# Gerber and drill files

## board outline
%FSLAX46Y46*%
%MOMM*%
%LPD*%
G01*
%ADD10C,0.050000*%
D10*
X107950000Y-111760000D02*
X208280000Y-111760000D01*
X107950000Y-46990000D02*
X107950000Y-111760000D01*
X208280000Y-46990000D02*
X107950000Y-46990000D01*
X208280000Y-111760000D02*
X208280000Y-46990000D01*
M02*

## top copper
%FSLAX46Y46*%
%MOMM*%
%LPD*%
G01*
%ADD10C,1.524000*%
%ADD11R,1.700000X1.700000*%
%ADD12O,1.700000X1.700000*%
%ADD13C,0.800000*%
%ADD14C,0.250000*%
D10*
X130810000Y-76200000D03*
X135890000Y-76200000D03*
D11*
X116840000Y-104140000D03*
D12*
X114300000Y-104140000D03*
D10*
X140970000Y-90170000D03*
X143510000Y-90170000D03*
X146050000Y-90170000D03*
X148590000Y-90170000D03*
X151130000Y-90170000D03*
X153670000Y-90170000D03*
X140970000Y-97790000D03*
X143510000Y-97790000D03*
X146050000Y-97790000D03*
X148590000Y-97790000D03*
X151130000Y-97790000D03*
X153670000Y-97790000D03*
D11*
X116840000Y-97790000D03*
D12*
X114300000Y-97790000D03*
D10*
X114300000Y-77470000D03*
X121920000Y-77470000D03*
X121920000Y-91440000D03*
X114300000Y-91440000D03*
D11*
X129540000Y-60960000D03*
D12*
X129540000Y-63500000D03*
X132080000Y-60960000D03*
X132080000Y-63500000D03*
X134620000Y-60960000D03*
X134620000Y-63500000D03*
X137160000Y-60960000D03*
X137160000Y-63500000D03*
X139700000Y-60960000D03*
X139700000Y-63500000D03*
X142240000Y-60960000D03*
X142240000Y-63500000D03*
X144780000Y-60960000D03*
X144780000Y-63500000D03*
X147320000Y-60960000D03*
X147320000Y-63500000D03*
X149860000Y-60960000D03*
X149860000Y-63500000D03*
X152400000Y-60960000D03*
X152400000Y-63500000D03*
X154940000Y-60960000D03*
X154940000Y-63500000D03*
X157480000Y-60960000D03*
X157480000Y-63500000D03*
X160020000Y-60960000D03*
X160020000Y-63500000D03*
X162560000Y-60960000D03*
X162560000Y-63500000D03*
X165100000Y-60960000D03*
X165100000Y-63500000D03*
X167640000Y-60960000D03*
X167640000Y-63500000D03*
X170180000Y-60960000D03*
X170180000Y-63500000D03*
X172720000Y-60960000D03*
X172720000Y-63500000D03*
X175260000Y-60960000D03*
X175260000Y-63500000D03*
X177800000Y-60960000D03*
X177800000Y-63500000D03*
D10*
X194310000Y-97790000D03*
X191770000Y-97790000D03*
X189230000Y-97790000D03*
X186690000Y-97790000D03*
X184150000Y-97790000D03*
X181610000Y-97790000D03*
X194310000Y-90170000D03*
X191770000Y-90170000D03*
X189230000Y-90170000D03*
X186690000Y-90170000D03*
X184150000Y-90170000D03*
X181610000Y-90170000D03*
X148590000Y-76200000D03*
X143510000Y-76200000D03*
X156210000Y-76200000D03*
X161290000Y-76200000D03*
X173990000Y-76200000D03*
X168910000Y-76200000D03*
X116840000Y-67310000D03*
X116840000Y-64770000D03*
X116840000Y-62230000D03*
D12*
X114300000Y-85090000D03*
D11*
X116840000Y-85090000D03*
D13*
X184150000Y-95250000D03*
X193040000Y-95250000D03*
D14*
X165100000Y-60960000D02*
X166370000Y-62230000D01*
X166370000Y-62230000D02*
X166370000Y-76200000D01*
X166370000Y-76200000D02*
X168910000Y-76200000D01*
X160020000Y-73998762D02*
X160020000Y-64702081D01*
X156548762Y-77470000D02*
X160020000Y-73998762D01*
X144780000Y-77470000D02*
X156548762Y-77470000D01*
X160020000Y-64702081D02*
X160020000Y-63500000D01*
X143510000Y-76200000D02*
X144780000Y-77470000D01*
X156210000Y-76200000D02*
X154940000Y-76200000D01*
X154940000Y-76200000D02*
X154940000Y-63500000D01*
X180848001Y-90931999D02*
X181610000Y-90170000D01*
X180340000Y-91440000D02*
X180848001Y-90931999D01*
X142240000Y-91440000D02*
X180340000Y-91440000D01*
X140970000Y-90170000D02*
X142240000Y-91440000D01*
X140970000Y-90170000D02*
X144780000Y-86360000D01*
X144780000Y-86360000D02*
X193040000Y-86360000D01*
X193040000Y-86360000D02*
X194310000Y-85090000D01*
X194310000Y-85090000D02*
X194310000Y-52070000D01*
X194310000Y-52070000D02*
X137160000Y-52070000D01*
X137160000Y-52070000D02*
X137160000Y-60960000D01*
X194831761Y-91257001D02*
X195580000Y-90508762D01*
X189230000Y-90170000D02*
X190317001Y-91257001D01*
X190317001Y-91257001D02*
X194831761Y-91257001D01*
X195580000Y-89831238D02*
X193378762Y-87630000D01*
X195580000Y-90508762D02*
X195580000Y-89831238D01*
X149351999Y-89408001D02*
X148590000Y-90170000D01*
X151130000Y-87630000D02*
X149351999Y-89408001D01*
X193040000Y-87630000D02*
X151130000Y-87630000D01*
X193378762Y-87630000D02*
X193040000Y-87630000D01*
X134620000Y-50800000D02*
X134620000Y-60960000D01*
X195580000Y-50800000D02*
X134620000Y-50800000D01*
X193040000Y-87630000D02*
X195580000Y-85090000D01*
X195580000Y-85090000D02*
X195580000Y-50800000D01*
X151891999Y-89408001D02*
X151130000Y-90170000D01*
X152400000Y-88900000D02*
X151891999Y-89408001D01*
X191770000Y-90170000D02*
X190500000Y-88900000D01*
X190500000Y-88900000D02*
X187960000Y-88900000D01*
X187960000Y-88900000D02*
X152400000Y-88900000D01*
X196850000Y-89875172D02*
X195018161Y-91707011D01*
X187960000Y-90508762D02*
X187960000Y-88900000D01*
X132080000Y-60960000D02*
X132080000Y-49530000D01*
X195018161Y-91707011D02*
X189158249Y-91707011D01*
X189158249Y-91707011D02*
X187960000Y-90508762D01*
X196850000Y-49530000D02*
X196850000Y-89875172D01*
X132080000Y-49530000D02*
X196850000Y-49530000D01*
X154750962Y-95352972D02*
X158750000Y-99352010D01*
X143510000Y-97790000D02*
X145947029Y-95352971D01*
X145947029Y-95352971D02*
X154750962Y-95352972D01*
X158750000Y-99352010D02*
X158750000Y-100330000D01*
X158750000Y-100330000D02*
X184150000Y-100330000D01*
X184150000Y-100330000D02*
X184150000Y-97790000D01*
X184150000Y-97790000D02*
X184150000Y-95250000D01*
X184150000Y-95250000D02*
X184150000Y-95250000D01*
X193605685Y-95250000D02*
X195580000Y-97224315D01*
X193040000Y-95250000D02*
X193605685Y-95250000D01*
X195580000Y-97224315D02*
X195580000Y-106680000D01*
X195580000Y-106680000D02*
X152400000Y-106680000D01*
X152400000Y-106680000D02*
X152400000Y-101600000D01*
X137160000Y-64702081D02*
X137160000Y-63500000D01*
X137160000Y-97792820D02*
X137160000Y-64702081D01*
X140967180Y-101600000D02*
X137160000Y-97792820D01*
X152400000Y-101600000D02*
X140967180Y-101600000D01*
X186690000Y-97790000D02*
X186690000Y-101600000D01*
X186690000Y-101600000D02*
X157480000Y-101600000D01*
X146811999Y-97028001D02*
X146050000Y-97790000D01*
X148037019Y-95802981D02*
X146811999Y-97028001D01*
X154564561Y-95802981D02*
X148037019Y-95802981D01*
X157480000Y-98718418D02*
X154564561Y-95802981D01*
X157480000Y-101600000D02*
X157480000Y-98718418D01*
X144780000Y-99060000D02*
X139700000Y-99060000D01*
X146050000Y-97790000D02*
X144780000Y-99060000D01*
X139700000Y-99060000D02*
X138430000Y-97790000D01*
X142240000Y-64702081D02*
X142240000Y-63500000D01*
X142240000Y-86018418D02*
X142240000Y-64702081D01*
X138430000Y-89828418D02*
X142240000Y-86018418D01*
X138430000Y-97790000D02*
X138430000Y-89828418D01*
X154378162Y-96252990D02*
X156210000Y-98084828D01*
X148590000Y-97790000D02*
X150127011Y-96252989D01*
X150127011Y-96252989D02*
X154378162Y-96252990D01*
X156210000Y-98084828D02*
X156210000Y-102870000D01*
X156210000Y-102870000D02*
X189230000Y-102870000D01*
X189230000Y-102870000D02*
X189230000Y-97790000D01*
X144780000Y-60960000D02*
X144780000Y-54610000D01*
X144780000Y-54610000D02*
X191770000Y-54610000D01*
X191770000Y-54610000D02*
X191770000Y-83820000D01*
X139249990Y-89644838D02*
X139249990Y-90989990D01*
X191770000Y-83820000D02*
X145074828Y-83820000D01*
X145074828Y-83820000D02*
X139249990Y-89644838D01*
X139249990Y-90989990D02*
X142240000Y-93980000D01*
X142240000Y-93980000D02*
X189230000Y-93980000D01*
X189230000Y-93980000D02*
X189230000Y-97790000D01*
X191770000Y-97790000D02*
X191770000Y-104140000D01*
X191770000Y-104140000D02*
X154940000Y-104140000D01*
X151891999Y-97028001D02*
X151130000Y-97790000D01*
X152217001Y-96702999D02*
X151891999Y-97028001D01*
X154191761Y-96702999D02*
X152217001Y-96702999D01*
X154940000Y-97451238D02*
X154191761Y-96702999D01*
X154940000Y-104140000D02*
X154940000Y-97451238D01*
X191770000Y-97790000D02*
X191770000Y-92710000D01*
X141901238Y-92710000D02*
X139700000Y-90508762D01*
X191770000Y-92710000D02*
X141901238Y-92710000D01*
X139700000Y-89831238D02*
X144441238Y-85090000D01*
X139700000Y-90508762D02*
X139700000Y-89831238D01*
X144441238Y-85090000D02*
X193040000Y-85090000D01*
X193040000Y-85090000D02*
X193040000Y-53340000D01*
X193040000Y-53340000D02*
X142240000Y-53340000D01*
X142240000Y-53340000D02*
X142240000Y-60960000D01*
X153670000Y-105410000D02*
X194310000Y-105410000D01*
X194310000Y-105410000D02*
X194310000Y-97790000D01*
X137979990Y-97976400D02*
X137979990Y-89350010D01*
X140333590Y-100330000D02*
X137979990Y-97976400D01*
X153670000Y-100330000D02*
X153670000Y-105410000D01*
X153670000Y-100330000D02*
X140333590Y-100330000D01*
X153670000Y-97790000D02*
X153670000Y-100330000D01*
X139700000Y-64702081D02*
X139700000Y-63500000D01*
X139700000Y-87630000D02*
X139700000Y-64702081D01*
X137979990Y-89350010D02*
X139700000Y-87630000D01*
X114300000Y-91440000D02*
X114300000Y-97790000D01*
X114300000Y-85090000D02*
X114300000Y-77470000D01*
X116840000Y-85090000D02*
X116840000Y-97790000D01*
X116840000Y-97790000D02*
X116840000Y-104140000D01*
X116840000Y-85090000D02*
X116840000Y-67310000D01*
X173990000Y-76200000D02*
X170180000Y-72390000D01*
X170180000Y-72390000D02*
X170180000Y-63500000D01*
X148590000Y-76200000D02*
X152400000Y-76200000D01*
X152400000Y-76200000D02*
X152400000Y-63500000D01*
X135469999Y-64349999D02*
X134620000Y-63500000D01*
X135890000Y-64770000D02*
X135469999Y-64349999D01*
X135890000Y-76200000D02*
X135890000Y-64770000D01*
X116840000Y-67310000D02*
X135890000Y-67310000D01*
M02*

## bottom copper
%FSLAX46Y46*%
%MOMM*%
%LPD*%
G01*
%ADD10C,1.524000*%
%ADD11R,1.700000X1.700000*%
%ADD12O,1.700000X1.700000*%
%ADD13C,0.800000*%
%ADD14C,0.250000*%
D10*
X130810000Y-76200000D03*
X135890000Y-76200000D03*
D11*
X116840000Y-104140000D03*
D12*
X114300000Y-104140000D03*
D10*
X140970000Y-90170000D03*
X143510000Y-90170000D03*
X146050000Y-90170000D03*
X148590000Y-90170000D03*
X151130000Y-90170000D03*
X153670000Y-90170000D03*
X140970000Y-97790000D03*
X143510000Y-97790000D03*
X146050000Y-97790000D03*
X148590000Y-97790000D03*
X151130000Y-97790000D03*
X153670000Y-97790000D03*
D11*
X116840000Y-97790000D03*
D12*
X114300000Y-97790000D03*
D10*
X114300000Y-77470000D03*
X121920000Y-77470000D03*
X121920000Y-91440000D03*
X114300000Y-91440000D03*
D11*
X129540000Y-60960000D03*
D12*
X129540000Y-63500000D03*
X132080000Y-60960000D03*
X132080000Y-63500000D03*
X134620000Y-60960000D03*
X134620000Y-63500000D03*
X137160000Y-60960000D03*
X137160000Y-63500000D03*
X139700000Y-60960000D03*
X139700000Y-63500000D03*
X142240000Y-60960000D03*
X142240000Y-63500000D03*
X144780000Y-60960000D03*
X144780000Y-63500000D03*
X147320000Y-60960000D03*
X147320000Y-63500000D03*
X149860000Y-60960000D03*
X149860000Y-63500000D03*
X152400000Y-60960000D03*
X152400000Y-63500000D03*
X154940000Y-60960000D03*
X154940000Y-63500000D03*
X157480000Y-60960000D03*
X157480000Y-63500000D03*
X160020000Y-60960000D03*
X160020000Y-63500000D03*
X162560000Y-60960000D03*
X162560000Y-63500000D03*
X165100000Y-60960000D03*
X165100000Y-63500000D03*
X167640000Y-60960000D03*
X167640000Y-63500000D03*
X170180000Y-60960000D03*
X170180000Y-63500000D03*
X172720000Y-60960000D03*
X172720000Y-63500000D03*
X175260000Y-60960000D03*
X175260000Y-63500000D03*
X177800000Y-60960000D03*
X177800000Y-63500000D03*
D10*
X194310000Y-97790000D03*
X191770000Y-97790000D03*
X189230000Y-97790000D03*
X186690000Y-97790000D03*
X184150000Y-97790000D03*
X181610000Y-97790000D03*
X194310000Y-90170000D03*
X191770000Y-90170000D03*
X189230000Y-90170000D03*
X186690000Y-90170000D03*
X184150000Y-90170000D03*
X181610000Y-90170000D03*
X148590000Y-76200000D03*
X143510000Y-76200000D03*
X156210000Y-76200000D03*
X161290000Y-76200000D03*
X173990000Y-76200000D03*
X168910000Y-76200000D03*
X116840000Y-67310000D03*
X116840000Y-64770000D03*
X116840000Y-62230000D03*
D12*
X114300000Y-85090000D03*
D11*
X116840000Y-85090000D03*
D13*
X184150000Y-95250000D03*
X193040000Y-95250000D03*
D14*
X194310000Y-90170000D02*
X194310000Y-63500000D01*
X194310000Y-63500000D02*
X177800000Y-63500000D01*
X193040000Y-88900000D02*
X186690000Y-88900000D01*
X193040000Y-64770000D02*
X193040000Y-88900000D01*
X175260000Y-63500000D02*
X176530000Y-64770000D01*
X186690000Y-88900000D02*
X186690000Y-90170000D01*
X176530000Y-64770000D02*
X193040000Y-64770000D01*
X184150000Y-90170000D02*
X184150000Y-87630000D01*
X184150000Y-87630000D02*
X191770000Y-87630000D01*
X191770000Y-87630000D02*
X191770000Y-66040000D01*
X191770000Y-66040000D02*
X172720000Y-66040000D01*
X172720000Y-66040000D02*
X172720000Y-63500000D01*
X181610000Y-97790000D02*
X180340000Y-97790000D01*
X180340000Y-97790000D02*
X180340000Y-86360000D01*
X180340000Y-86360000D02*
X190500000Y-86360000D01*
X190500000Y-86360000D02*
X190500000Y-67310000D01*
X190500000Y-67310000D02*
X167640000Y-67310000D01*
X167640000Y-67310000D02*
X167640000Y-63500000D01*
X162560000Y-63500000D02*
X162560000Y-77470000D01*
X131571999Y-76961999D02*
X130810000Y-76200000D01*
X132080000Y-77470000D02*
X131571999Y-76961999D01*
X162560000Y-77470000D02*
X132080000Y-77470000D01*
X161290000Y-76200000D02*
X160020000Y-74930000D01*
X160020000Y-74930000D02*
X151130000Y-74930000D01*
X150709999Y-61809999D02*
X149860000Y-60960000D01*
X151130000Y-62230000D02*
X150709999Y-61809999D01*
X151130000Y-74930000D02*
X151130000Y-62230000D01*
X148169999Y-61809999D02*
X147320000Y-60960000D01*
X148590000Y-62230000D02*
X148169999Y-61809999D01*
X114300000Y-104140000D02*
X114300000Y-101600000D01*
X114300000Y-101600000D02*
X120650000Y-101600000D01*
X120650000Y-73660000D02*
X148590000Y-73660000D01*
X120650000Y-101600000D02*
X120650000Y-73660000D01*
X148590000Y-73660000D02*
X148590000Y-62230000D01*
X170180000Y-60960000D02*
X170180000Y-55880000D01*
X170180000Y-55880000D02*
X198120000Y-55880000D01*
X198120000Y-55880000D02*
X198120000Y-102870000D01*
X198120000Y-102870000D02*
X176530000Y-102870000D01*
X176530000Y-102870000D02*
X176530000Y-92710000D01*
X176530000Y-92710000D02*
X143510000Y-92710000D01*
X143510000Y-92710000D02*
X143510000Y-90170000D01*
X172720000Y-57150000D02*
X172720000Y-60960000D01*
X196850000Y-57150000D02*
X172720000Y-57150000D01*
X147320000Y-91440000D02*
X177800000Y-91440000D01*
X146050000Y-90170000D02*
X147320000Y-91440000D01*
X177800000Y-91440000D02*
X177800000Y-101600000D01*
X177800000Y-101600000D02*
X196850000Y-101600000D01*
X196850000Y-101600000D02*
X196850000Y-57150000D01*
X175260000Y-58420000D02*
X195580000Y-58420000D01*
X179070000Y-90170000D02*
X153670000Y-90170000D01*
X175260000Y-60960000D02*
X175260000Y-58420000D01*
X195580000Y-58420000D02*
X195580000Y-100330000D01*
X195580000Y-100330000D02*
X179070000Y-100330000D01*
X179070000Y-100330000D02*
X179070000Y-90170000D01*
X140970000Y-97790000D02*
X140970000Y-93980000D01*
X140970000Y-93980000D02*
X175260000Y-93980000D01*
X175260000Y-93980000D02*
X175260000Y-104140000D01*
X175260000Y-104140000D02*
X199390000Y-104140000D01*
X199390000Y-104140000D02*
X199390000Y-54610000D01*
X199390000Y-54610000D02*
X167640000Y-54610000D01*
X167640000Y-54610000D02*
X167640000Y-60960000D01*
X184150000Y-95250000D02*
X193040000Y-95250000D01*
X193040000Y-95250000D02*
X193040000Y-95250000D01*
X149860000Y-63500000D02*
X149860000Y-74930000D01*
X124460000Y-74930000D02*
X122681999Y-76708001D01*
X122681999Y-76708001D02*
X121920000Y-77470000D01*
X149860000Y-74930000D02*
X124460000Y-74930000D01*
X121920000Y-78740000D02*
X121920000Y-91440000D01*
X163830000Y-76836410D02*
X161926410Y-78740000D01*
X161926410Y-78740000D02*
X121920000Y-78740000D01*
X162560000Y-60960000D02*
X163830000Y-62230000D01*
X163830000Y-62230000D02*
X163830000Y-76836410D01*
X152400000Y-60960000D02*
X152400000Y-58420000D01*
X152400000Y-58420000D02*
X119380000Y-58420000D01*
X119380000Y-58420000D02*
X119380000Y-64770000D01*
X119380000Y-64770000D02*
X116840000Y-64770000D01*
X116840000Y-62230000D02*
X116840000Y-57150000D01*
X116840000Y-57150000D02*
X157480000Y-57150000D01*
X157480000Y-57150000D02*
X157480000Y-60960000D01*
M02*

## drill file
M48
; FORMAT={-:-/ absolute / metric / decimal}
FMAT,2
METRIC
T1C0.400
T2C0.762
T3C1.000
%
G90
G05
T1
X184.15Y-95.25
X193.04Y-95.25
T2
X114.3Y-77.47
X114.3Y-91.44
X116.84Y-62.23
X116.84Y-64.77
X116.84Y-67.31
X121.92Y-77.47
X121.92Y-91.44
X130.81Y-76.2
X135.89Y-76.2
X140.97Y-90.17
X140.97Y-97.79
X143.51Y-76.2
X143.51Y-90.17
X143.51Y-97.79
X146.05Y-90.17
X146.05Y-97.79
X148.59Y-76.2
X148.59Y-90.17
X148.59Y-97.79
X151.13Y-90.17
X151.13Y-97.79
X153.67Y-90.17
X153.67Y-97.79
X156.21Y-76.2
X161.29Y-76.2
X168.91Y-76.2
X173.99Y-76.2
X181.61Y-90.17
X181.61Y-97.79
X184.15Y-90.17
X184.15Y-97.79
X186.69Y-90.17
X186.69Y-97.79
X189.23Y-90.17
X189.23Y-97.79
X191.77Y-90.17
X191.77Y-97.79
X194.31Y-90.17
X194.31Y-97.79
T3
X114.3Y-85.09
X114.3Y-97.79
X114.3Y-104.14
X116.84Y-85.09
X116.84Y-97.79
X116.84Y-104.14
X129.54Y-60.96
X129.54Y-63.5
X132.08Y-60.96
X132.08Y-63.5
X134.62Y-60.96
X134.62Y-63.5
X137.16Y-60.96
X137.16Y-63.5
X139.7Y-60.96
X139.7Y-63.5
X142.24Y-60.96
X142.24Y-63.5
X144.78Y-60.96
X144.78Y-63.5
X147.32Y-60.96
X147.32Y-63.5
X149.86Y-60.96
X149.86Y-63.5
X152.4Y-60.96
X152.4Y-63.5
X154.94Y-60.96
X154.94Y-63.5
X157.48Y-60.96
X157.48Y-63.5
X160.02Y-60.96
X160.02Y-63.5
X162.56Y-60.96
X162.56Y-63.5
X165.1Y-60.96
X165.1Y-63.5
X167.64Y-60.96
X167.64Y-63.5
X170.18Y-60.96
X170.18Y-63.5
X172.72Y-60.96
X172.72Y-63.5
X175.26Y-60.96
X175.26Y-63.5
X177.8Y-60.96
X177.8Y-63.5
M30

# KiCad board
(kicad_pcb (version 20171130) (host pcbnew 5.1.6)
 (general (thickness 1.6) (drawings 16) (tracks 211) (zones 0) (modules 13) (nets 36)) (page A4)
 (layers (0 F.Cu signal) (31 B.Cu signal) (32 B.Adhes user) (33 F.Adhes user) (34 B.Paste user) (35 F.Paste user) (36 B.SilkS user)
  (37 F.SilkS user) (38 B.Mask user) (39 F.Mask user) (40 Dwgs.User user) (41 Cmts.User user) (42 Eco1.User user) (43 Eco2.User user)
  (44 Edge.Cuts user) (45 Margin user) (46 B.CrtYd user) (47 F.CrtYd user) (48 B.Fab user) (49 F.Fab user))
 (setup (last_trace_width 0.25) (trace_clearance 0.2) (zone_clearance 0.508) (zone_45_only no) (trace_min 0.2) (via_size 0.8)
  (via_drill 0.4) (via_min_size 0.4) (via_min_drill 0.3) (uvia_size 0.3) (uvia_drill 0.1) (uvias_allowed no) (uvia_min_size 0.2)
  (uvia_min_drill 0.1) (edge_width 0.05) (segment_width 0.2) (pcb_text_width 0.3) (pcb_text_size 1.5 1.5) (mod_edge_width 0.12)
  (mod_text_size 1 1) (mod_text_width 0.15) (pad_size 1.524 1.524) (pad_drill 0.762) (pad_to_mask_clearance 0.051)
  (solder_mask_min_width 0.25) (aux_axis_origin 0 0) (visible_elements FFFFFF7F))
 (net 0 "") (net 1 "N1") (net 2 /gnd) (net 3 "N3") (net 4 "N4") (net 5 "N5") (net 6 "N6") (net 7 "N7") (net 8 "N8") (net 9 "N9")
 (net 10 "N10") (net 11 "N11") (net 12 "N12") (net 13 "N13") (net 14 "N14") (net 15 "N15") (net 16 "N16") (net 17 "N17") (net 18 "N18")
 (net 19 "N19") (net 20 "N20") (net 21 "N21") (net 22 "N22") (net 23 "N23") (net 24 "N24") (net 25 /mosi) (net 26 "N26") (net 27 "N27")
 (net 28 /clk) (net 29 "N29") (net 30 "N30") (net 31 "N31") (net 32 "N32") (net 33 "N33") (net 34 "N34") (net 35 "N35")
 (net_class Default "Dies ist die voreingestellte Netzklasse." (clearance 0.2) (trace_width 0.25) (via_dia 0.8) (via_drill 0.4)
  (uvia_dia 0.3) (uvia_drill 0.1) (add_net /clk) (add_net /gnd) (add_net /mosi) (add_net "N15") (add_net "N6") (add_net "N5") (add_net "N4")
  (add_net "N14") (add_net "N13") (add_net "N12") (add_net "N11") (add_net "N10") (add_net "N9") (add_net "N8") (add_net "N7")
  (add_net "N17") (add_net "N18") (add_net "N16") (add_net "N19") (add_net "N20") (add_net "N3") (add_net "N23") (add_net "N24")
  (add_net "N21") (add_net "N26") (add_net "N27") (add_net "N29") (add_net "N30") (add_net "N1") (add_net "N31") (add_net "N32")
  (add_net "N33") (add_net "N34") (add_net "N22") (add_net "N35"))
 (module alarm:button (layer B.Cu) (at 133.35 76.2)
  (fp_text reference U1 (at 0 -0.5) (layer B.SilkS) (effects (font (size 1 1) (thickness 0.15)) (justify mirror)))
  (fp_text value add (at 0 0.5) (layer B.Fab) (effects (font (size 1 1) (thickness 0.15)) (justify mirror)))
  (pad 1 thru_hole circle (at -2.54 0) (size 1.524 1.524) (drill 0.762) (layers *.Cu *.Mask) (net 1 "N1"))
  (pad 2 thru_hole circle (at 2.54 0) (size 1.524 1.524) (drill 0.762) (layers *.Cu *.Mask) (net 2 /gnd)))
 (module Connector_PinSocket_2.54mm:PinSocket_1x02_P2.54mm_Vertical (layer B.Cu) (at 116.84 104.14 90)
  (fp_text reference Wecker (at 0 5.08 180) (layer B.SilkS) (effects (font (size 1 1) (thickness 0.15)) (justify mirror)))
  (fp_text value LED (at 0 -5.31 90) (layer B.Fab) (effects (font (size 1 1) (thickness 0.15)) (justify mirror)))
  (pad 1 thru_hole rect (at 0 0 90) (size 1.7 1.7) (drill 1) (layers *.Cu *.Mask) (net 2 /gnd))
  (pad 2 thru_hole oval (at 0 -2.54 90) (size 1.7 1.7) (drill 1) (layers *.Cu *.Mask) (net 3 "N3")))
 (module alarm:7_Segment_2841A (layer B.Cu) (at 146.05 95.25 180)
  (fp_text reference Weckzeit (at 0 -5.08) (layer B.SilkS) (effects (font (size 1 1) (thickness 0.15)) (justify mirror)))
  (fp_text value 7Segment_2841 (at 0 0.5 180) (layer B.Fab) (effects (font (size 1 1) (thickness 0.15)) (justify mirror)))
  (pad 12 thru_hole circle (at 5.08 5.08 180) (size 1.524 1.524) (drill 0.762) (layers *.Cu *.Mask) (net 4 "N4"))
  (pad 11 thru_hole circle (at 2.54 5.08 180) (size 1.524 1.524) (drill 0.762) (layers *.Cu *.Mask) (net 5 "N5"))
  (pad 10 thru_hole circle (at 0 5.08 180) (size 1.524 1.524) (drill 0.762) (layers *.Cu *.Mask) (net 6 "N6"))
  (pad 9 thru_hole circle (at -2.54 5.08 180) (size 1.524 1.524) (drill 0.762) (layers *.Cu *.Mask) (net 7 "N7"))
  (pad 8 thru_hole circle (at -5.08 5.08 180) (size 1.524 1.524) (drill 0.762) (layers *.Cu *.Mask) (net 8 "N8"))
  (pad 7 thru_hole circle (at -7.62 5.08 180) (size 1.524 1.524) (drill 0.762) (layers *.Cu *.Mask) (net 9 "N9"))
  (pad 6 thru_hole circle (at 5.08 -2.54 180) (size 1.524 1.524) (drill 0.762) (layers *.Cu *.Mask) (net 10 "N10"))
  (pad 5 thru_hole circle (at 2.54 -2.54 180) (size 1.524 1.524) (drill 0.762) (layers *.Cu *.Mask) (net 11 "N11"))
  (pad 4 thru_hole circle (at 0 -2.54 180) (size 1.524 1.524) (drill 0.762) (layers *.Cu *.Mask) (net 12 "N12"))
  (pad 3 thru_hole circle (at -2.54 -2.54 180) (size 1.524 1.524) (drill 0.762) (layers *.Cu *.Mask) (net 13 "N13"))
  (pad 2 thru_hole circle (at -5.08 -2.54 180) (size 1.524 1.524) (drill 0.762) (layers *.Cu *.Mask) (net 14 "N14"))
  (pad 1 thru_hole circle (at -7.62 -2.54 180) (size 1.524 1.524) (drill 0.762) (layers *.Cu *.Mask) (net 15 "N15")))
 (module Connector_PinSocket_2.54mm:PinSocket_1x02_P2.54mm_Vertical (layer B.Cu) (at 116.84 97.79 90)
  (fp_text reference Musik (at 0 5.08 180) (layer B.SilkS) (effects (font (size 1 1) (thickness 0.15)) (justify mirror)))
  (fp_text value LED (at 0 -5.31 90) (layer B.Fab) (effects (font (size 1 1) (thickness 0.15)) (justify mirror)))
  (pad 1 thru_hole rect (at 0 0 90) (size 1.7 1.7) (drill 1) (layers *.Cu *.Mask) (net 2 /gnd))
  (pad 2 thru_hole oval (at 0 -2.54 90) (size 1.7 1.7) (drill 1) (layers *.Cu *.Mask) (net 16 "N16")))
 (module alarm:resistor (layer B.Cu) (at 119.38 77.47)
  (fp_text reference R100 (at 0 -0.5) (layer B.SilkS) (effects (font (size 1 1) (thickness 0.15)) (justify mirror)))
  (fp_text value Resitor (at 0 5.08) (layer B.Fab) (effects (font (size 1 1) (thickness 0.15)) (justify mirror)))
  (pad 1 thru_hole circle (at -5.08 0) (size 1.524 1.524) (drill 0.762) (layers *.Cu *.Mask) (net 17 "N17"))
  (pad 2 thru_hole circle (at 2.54 0) (size 1.524 1.524) (drill 0.762) (layers *.Cu *.Mask) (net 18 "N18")))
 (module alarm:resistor (layer B.Cu) (at 119.38 91.44)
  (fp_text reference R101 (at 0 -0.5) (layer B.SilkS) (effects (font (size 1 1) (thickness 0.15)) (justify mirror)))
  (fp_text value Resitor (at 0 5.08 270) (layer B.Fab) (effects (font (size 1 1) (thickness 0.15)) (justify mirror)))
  (pad 2 thru_hole circle (at 2.54 0) (size 1.524 1.524) (drill 0.762) (layers *.Cu *.Mask) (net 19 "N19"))
  (pad 1 thru_hole circle (at -5.08 0) (size 1.524 1.524) (drill 0.762) (layers *.Cu *.Mask) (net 16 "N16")))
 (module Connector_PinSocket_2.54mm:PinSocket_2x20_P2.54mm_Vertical (layer F.Cu) (at 129.54 60.96 90)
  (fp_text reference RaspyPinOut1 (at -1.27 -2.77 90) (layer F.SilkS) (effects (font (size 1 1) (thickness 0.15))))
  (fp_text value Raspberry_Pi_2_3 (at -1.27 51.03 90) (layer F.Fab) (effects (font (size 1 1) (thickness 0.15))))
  (pad 1 thru_hole rect (at 0 0 90) (size 1.7 1.7) (drill 1) (layers *.Cu *.Mask) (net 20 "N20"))
  (pad 2 thru_hole oval (at -2.54 0 90) (size 1.7 1.7) (drill 1) (layers *.Cu *.Mask) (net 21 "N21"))
  (pad 3 thru_hole oval (at 0 2.54 90) (size 1.7 1.7) (drill 1) (layers *.Cu *.Mask) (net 8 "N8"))
  (pad 4 thru_hole oval (at -2.54 2.54 90) (size 1.7 1.7) (drill 1) (layers *.Cu *.Mask) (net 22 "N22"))
  (pad 5 thru_hole oval (at 0 5.08 90) (size 1.7 1.7) (drill 1) (layers *.Cu *.Mask) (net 7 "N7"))
  (pad 6 thru_hole oval (at -2.54 5.08 90) (size 1.7 1.7) (drill 1) (layers *.Cu *.Mask) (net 2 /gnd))
  (pad 7 thru_hole oval (at 0 7.62 90) (size 1.7 1.7) (drill 1) (layers *.Cu *.Mask) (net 4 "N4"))
  (pad 8 thru_hole oval (at -2.54 7.62 90) (size 1.7 1.7) (drill 1) (layers *.Cu *.Mask) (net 11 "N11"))
  (pad 9 thru_hole oval (at 0 10.16 90) (size 1.7 1.7) (drill 1) (layers *.Cu *.Mask) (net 2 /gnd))
  (pad 10 thru_hole oval (at -2.54 10.16 90) (size 1.7 1.7) (drill 1) (layers *.Cu *.Mask) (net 15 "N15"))
  (pad 11 thru_hole oval (at 0 12.7 90) (size 1.7 1.7) (drill 1) (layers *.Cu *.Mask) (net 14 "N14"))
  (pad 12 thru_hole oval (at -2.54 12.7 90) (size 1.7 1.7) (drill 1) (layers *.Cu *.Mask) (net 12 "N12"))
  (pad 13 thru_hole oval (at 0 15.24 90) (size 1.7 1.7) (drill 1) (layers *.Cu *.Mask) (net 13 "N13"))
  (pad 14 thru_hole oval (at -2.54 15.24 90) (size 1.7 1.7) (drill 1) (layers *.Cu *.Mask) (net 2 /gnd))
  (pad 15 thru_hole oval (at 0 17.78 90) (size 1.7 1.7) (drill 1) (layers *.Cu *.Mask) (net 3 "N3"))
  (pad 16 thru_hole oval (at -2.54 17.78 90) (size 1.7 1.7) (drill 1) (layers *.Cu *.Mask) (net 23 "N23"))
  (pad 17 thru_hole oval (at 0 20.32 90) (size 1.7 1.7) (drill 1) (layers *.Cu *.Mask) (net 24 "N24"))
  (pad 18 thru_hole oval (at -2.54 20.32 90) (size 1.7 1.7) (drill 1) (layers *.Cu *.Mask) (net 18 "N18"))
  (pad 19 thru_hole oval (at 0 22.86 90) (size 1.7 1.7) (drill 1) (layers *.Cu *.Mask) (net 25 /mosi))
  (pad 20 thru_hole oval (at -2.54 22.86 90) (size 1.7 1.7) (drill 1) (layers *.Cu *.Mask) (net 2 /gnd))
  (pad 21 thru_hole oval (at 0 25.4 90) (size 1.7 1.7) (drill 1) (layers *.Cu *.Mask) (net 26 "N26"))
  (pad 22 thru_hole oval (at -2.54 25.4 90) (size 1.7 1.7) (drill 1) (layers *.Cu *.Mask) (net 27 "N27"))
  (pad 23 thru_hole oval (at 0 27.94 90) (size 1.7 1.7) (drill 1) (layers *.Cu *.Mask) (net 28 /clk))
  (pad 24 thru_hole oval (at -2.54 27.94 90) (size 1.7 1.7) (drill 1) (layers *.Cu *.Mask) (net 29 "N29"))
  (pad 25 thru_hole oval (at 0 30.48 90) (size 1.7 1.7) (drill 1) (layers *.Cu *.Mask) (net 2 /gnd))
  (pad 26 thru_hole oval (at -2.54 30.48 90) (size 1.7 1.7) (drill 1) (layers *.Cu *.Mask) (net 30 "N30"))
  (pad 27 thru_hole oval (at 0 33.02 90) (size 1.7 1.7) (drill 1) (layers *.Cu *.Mask) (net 19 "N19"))
  (pad 28 thru_hole oval (at -2.54 33.02 90) (size 1.7 1.7) (drill 1) (layers *.Cu *.Mask) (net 1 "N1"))
  (pad 29 thru_hole oval (at 0 35.56 90) (size 1.7 1.7) (drill 1) (layers *.Cu *.Mask) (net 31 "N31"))
  (pad 30 thru_hole oval (at -2.54 35.56 90) (size 1.7 1.7) (drill 1) (layers *.Cu *.Mask) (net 2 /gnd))
  (pad 31 thru_hole oval (at 0 38.1 90) (size 1.7 1.7) (drill 1) (layers *.Cu *.Mask) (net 10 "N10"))
  (pad 32 thru_hole oval (at -2.54 38.1 90) (size 1.7 1.7) (drill 1) (layers *.Cu *.Mask) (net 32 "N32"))
  (pad 33 thru_hole oval (at 0 40.64 90) (size 1.7 1.7) (drill 1) (layers *.Cu *.Mask) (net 5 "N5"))
  (pad 34 thru_hole oval (at -2.54 40.64 90) (size 1.7 1.7) (drill 1) (layers *.Cu *.Mask) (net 2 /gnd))
  (pad 35 thru_hole oval (at 0 43.18 90) (size 1.7 1.7) (drill 1) (layers *.Cu *.Mask) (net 6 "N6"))
  (pad 36 thru_hole oval (at -2.54 43.18 90) (size 1.7 1.7) (drill 1) (layers *.Cu *.Mask) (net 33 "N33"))
  (pad 37 thru_hole oval (at 0 45.72 90) (size 1.7 1.7) (drill 1) (layers *.Cu *.Mask) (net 9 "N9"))
  (pad 38 thru_hole oval (at -2.54 45.72 90) (size 1.7 1.7) (drill 1) (layers *.Cu *.Mask) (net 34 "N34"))
  (pad 39 thru_hole oval (at 0 48.26 90) (size 1.7 1.7) (drill 1) (layers *.Cu *.Mask) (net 2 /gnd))
  (pad 40 thru_hole oval (at -2.54 48.26 90) (size 1.7 1.7) (drill 1) (layers *.Cu *.Mask) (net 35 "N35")))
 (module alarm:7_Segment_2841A (layer B.Cu) (at 186.69 95.25 180)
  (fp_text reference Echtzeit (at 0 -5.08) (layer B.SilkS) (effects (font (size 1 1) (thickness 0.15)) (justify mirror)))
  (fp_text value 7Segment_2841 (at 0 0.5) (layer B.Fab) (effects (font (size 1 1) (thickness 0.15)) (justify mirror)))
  (pad 1 thru_hole circle (at -7.62 -2.54 180) (size 1.524 1.524) (drill 0.762) (layers *.Cu *.Mask) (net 15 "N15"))
  (pad 2 thru_hole circle (at -5.08 -2.54 180) (size 1.524 1.524) (drill 0.762) (layers *.Cu *.Mask) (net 14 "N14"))
  (pad 3 thru_hole circle (at -2.54 -2.54 180) (size 1.524 1.524) (drill 0.762) (layers *.Cu *.Mask) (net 13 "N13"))
  (pad 4 thru_hole circle (at 0 -2.54 180) (size 1.524 1.524) (drill 0.762) (layers *.Cu *.Mask) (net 12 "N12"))
  (pad 5 thru_hole circle (at 2.54 -2.54 180) (size 1.524 1.524) (drill 0.762) (layers *.Cu *.Mask) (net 11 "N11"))
  (pad 6 thru_hole circle (at 5.08 -2.54 180) (size 1.524 1.524) (drill 0.762) (layers *.Cu *.Mask) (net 32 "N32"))
  (pad 7 thru_hole circle (at -7.62 5.08 180) (size 1.524 1.524) (drill 0.762) (layers *.Cu *.Mask) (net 35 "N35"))
  (pad 8 thru_hole circle (at -5.08 5.08 180) (size 1.524 1.524) (drill 0.762) (layers *.Cu *.Mask) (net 8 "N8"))
  (pad 9 thru_hole circle (at -2.54 5.08 180) (size 1.524 1.524) (drill 0.762) (layers *.Cu *.Mask) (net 7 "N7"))
  (pad 10 thru_hole circle (at 0 5.08 180) (size 1.524 1.524) (drill 0.762) (layers *.Cu *.Mask) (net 34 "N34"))
  (pad 11 thru_hole circle (at 2.54 5.08 180) (size 1.524 1.524) (drill 0.762) (layers *.Cu *.Mask) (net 33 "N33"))
  (pad 12 thru_hole circle (at 5.08 5.08 180) (size 1.524 1.524) (drill 0.762) (layers *.Cu *.Mask) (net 4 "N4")))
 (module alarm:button (layer B.Cu) (at 146.05 76.2)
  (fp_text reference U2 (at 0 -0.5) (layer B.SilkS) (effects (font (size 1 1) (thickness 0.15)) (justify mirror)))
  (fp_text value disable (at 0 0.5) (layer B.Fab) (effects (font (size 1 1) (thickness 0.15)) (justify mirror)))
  (pad 2 thru_hole circle (at 2.54 0) (size 1.524 1.524) (drill 0.762) (layers *.Cu *.Mask) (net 2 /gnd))
  (pad 1 thru_hole circle (at -2.54 0) (size 1.524 1.524) (drill 0.762) (layers *.Cu *.Mask) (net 30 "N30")))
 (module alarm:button (layer B.Cu) (at 158.75 76.2)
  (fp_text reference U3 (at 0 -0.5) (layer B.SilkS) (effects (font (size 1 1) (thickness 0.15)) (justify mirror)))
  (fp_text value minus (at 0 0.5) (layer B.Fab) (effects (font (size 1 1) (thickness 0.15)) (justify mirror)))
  (pad 1 thru_hole circle (at -2.54 0) (size 1.524 1.524) (drill 0.762) (layers *.Cu *.Mask) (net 27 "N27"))
  (pad 2 thru_hole circle (at 2.54 0) (size 1.524 1.524) (drill 0.762) (layers *.Cu *.Mask) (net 24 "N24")))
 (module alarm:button (layer B.Cu) (at 171.45 76.2)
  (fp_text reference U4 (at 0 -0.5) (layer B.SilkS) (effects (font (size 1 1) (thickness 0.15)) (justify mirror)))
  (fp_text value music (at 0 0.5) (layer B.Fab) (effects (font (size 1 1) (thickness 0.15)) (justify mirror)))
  (pad 2 thru_hole circle (at 2.54 0) (size 1.524 1.524) (drill 0.762) (layers *.Cu *.Mask) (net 2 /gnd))
  (pad 1 thru_hole circle (at -2.54 0) (size 1.524 1.524) (drill 0.762) (layers *.Cu *.Mask) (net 31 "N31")))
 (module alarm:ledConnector (layer B.Cu) (at 116.84 62.23 90)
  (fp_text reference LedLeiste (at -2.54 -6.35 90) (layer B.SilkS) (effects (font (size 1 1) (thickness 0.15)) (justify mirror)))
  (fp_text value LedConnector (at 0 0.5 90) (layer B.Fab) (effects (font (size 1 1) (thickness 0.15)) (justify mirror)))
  (pad 1 thru_hole circle (at -5.08 0 90) (size 1.524 1.524) (drill 0.762) (layers *.Cu *.Mask) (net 2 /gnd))
  (pad 2 thru_hole circle (at -2.54 0 90) (size 1.524 1.524) (drill 0.762) (layers *.Cu *.Mask) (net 25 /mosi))
  (pad 3 thru_hole circle (at 0 0 90) (size 1.524 1.524) (drill 0.762) (layers *.Cu *.Mask) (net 28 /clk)))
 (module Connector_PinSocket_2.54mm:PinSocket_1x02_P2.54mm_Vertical (layer B.Cu) (at 116.84 85.09 90)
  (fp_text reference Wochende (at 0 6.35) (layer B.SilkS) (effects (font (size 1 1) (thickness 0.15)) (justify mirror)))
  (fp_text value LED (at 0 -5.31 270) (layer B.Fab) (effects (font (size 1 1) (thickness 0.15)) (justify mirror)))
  (pad 2 thru_hole oval (at 0 -2.54 90) (size 1.7 1.7) (drill 1) (layers *.Cu *.Mask) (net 17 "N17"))
  (pad 1 thru_hole rect (at 0 0 90) (size 1.7 1.7) (drill 1) (layers *.Cu *.Mask) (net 2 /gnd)))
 (gr_line (start 107.95 111.76) (end 208.28 111.76) (layer Edge.Cuts) (width 0.05))
 (gr_line (start 107.95 46.99) (end 107.95 111.76) (layer Edge.Cuts) (width 0.05))
 (gr_line (start 208.28 46.99) (end 107.95 46.99) (layer Edge.Cuts) (width 0.05))
 (gr_line (start 208.28 111.76) (end 208.28 46.99) (layer Edge.Cuts) (width 0.05))
 (segment (start 194.31 90.17) (end 194.31 63.5) (width 0.25) (layer B.Cu) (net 35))
 (segment (start 194.31 63.5) (end 177.8 63.5) (width 0.25) (layer B.Cu) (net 35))
 (segment (start 193.04 88.9) (end 186.69 88.9) (width 0.25) (layer B.Cu) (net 34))
 (segment (start 193.04 64.77) (end 193.04 88.9) (width 0.25) (layer B.Cu) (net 34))
 (segment (start 175.26 63.5) (end 176.53 64.77) (width 0.25) (layer B.Cu) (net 34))
 (segment (start 186.69 88.9) (end 186.69 90.17) (width 0.25) (layer B.Cu) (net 34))
 (segment (start 176.53 64.77) (end 193.04 64.77) (width 0.25) (layer B.Cu) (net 34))
 (segment (start 184.15 90.17) (end 184.15 87.63) (width 0.25) (layer B.Cu) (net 33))
 (segment (start 184.15 87.63) (end 191.77 87.63) (width 0.25) (layer B.Cu) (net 33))
 (segment (start 191.77 87.63) (end 191.77 66.04) (width 0.25) (layer B.Cu) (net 33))
 (segment (start 191.77 66.04) (end 172.72 66.04) (width 0.25) (layer B.Cu) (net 33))
 (segment (start 172.72 66.04) (end 172.72 63.5) (width 0.25) (layer B.Cu) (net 33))
 (segment (start 181.61 97.79) (end 180.34 97.79) (width 0.25) (layer B.Cu) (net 32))
 (segment (start 180.34 97.79) (end 180.34 86.36) (width 0.25) (layer B.Cu) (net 32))
 (segment (start 180.34 86.36) (end 190.5 86.36) (width 0.25) (layer B.Cu) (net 32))
 (segment (start 190.5 86.36) (end 190.5 67.31) (width 0.25) (layer B.Cu) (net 32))
 (segment (start 190.5 67.31) (end 167.64 67.31) (width 0.25) (layer B.Cu) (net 32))
 (segment (start 167.64 67.31) (end 167.64 63.5) (width 0.25) (layer B.Cu) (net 32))
 (segment (start 165.1 60.96) (end 166.37 62.23) (width 0.25) (layer F.Cu) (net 31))
 (segment (start 166.37 62.23) (end 166.37 76.2) (width 0.25) (layer F.Cu) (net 31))
 (segment (start 166.37 76.2) (end 168.91 76.2) (width 0.25) (layer F.Cu) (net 31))
 (segment (start 162.56 63.5) (end 162.56 77.47) (width 0.25) (layer B.Cu) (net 1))
 (segment (start 131.571999 76.961999) (end 130.81 76.2) (width 0.25) (layer B.Cu) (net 1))
 (segment (start 132.08 77.47) (end 131.571999 76.961999) (width 0.25) (layer B.Cu) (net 1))
 (segment (start 162.56 77.47) (end 132.08 77.47) (width 0.25) (layer B.Cu) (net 1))
 (segment (start 160.02 73.998762) (end 160.02 64.702081) (width 0.25) (layer F.Cu) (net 30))
 (segment (start 156.548762 77.47) (end 160.02 73.998762) (width 0.25) (layer F.Cu) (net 30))
 (segment (start 144.78 77.47) (end 156.548762 77.47) (width 0.25) (layer F.Cu) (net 30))
 (segment (start 160.02 64.702081) (end 160.02 63.5) (width 0.25) (layer F.Cu) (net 30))
 (segment (start 143.51 76.2) (end 144.78 77.47) (width 0.25) (layer F.Cu) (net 30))
 (segment (start 156.21 76.2) (end 154.94 76.2) (width 0.25) (layer F.Cu) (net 27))
 (segment (start 154.94 76.2) (end 154.94 63.5) (width 0.25) (layer F.Cu) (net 27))
 (segment (start 161.29 76.2) (end 160.02 74.93) (width 0.25) (layer B.Cu) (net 24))
 (segment (start 160.02 74.93) (end 151.13 74.93) (width 0.25) (layer B.Cu) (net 24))
 (segment (start 150.709999 61.809999) (end 149.86 60.96) (width 0.25) (layer B.Cu) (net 24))
 (segment (start 151.13 62.23) (end 150.709999 61.809999) (width 0.25) (layer B.Cu) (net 24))
 (segment (start 151.13 74.93) (end 151.13 62.23) (width 0.25) (layer B.Cu) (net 24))
 (segment (start 148.169999 61.809999) (end 147.32 60.96) (width 0.25) (layer B.Cu) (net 3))
 (segment (start 148.59 62.23) (end 148.169999 61.809999) (width 0.25) (layer B.Cu) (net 3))
 (segment (start 114.3 104.14) (end 114.3 101.6) (width 0.25) (layer B.Cu) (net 3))
 (segment (start 114.3 101.6) (end 120.65 101.6) (width 0.25) (layer B.Cu) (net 3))
 (segment (start 120.65 73.66) (end 148.59 73.66) (width 0.25) (layer B.Cu) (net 3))
 (segment (start 120.65 101.6) (end 120.65 73.66) (width 0.25) (layer B.Cu) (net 3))
 (segment (start 148.59 73.66) (end 148.59 62.23) (width 0.25) (layer B.Cu) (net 3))
 (segment (start 180.848001 90.931999) (end 181.61 90.17) (width 0.25) (layer F.Cu) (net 4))
 (segment (start 180.34 91.44) (end 180.848001 90.931999) (width 0.25) (layer F.Cu) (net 4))
 (segment (start 142.24 91.44) (end 180.34 91.44) (width 0.25) (layer F.Cu) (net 4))
 (segment (start 140.97 90.17) (end 142.24 91.44) (width 0.25) (layer F.Cu) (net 4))
 (segment (start 140.97 90.17) (end 144.78 86.36) (width 0.25) (layer F.Cu) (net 4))
 (segment (start 144.78 86.36) (end 193.04 86.36) (width 0.25) (layer F.Cu) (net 4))
 (segment (start 193.04 86.36) (end 194.31 85.09) (width 0.25) (layer F.Cu) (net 4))
 (segment (start 194.31 85.09) (end 194.31 52.07) (width 0.25) (layer F.Cu) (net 4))
 (segment (start 194.31 52.07) (end 137.16 52.07) (width 0.25) (layer F.Cu) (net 4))
 (segment (start 137.16 52.07) (end 137.16 60.96) (width 0.25) (layer F.Cu) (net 4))
 (segment (start 170.18 60.96) (end 170.18 55.88) (width 0.25) (layer B.Cu) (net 5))
 (segment (start 170.18 55.88) (end 198.12 55.88) (width 0.25) (layer B.Cu) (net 5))
 (segment (start 198.12 55.88) (end 198.12 102.87) (width 0.25) (layer B.Cu) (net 5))
 (segment (start 198.12 102.87) (end 176.53 102.87) (width 0.25) (layer B.Cu) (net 5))
 (segment (start 176.53 102.87) (end 176.53 92.71) (width 0.25) (layer B.Cu) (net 5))
 (segment (start 176.53 92.71) (end 143.51 92.71) (width 0.25) (layer B.Cu) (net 5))
 (segment (start 143.51 92.71) (end 143.51 90.17) (width 0.25) (layer B.Cu) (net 5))
 (segment (start 172.72 57.15) (end 172.72 60.96) (width 0.25) (layer B.Cu) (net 6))
 (segment (start 196.85 57.15) (end 172.72 57.15) (width 0.25) (layer B.Cu) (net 6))
 (segment (start 147.32 91.44) (end 177.8 91.44) (width 0.25) (layer B.Cu) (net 6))
 (segment (start 146.05 90.17) (end 147.32 91.44) (width 0.25) (layer B.Cu) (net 6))
 (segment (start 177.8 91.44) (end 177.8 101.6) (width 0.25) (layer B.Cu) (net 6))
 (segment (start 177.8 101.6) (end 196.85 101.6) (width 0.25) (layer B.Cu) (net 6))
 (segment (start 196.85 101.6) (end 196.85 57.15) (width 0.25) (layer B.Cu) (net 6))
 (segment (start 194.831761 91.257001) (end 195.58 90.508762) (width 0.25) (layer F.Cu) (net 7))
 (segment (start 189.23 90.17) (end 190.317001 91.257001) (width 0.25) (layer F.Cu) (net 7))
 (segment (start 190.317001 91.257001) (end 194.831761 91.257001) (width 0.25) (layer F.Cu) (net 7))
 (segment (start 195.58 89.831238) (end 193.378762 87.63) (width 0.25) (layer F.Cu) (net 7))
 (segment (start 195.58 90.508762) (end 195.58 89.831238) (width 0.25) (layer F.Cu) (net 7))
 (segment (start 149.351999 89.408001) (end 148.59 90.17) (width 0.25) (layer F.Cu) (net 7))
 (segment (start 151.13 87.63) (end 149.351999 89.408001) (width 0.25) (layer F.Cu) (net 7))
 (segment (start 193.04 87.63) (end 151.13 87.63) (width 0.25) (layer F.Cu) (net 7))
 (segment (start 193.378762 87.63) (end 193.04 87.63) (width 0.25) (layer F.Cu) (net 7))
 (segment (start 134.62 50.8) (end 134.62 60.96) (width 0.25) (layer F.Cu) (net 7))
 (segment (start 195.58 50.8) (end 134.62 50.8) (width 0.25) (layer F.Cu) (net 7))
 (segment (start 193.04 87.63) (end 195.58 85.09) (width 0.25) (layer F.Cu) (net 7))
 (segment (start 195.58 85.09) (end 195.58 50.8) (width 0.25) (layer F.Cu) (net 7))
 (segment (start 151.891999 89.408001) (end 151.13 90.17) (width 0.25) (layer F.Cu) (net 8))
 (segment (start 152.4 88.9) (end 151.891999 89.408001) (width 0.25) (layer F.Cu) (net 8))
 (segment (start 191.77 90.17) (end 190.5 88.9) (width 0.25) (layer F.Cu) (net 8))
 (segment (start 190.5 88.9) (end 187.96 88.9) (width 0.25) (layer F.Cu) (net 8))
 (segment (start 187.96 88.9) (end 152.4 88.9) (width 0.25) (layer F.Cu) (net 8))
 (segment (start 196.85 89.875172) (end 195.018161 91.707011) (width 0.25) (layer F.Cu) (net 8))
 (segment (start 187.96 90.508762) (end 187.96 88.9) (width 0.25) (layer F.Cu) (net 8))
 (segment (start 132.08 60.96) (end 132.08 49.53) (width 0.25) (layer F.Cu) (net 8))
 (segment (start 195.018161 91.707011) (end 189.158249 91.707011) (width 0.25) (layer F.Cu) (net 8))
 (segment (start 189.158249 91.707011) (end 187.96 90.508762) (width 0.25) (layer F.Cu) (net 8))
 (segment (start 196.85 49.53) (end 196.85 89.875172) (width 0.25) (layer F.Cu) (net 8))
 (segment (start 132.08 49.53) (end 196.85 49.53) (width 0.25) (layer F.Cu) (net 8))
 (segment (start 175.26 58.42) (end 195.58 58.42) (width 0.25) (layer B.Cu) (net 9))
 (segment (start 179.07 90.17) (end 153.67 90.17) (width 0.25) (layer B.Cu) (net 9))
 (segment (start 175.26 60.96) (end 175.26 58.42) (width 0.25) (layer B.Cu) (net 9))
 (segment (start 195.58 58.42) (end 195.58 100.33) (width 0.25) (layer B.Cu) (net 9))
 (segment (start 195.58 100.33) (end 179.07 100.33) (width 0.25) (layer B.Cu) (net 9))
 (segment (start 179.07 100.33) (end 179.07 90.17) (width 0.25) (layer B.Cu) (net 9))
 (segment (start 140.97 97.79) (end 140.97 93.98) (width 0.25) (layer B.Cu) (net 10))
 (segment (start 140.97 93.98) (end 175.26 93.98) (width 0.25) (layer B.Cu) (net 10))
 (segment (start 175.26 93.98) (end 175.26 104.14) (width 0.25) (layer B.Cu) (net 10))
 (segment (start 175.26 104.14) (end 199.39 104.14) (width 0.25) (layer B.Cu) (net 10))
 (segment (start 199.39 104.14) (end 199.39 54.61) (width 0.25) (layer B.Cu) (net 10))
 (segment (start 199.39 54.61) (end 167.64 54.61) (width 0.25) (layer B.Cu) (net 10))
 (segment (start 167.64 54.61) (end 167.64 60.96) (width 0.25) (layer B.Cu) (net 10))
 (segment (start 154.750962 95.352972) (end 158.75 99.35201) (width 0.25) (layer F.Cu) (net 11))
 (segment (start 143.51 97.79) (end 145.947029 95.352971) (width 0.25) (layer F.Cu) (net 11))
 (segment (start 145.947029 95.352971) (end 154.750962 95.352972) (width 0.25) (layer F.Cu) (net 11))
 (segment (start 158.75 99.35201) (end 158.75 100.33) (width 0.25) (layer F.Cu) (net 11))
 (segment (start 158.75 100.33) (end 184.15 100.33) (width 0.25) (layer F.Cu) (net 11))
 (segment (start 184.15 100.33) (end 184.15 97.79) (width 0.25) (layer F.Cu) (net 11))
 (segment (start 184.15 97.79) (end 184.15 95.25) (width 0.25) (layer F.Cu) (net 11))
 (segment (start 184.15 95.25) (end 184.15 95.25) (width 0.25) (layer F.Cu) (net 11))
 (via (at 184.15 95.25) (size 0.8) (drill 0.4) (layers F.Cu B.Cu) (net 11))
 (segment (start 184.15 95.25) (end 193.04 95.25) (width 0.25) (layer B.Cu) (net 11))
 (segment (start 193.04 95.25) (end 193.04 95.25) (width 0.25) (layer B.Cu) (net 11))
 (via (at 193.04 95.25) (size 0.8) (drill 0.4) (layers F.Cu B.Cu) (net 11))
 (segment (start 193.605685 95.25) (end 195.58 97.224315) (width 0.25) (layer F.Cu) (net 11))
 (segment (start 193.04 95.25) (end 193.605685 95.25) (width 0.25) (layer F.Cu) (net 11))
 (segment (start 195.58 97.224315) (end 195.58 106.68) (width 0.25) (layer F.Cu) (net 11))
 (segment (start 195.58 106.68) (end 152.4 106.68) (width 0.25) (layer F.Cu) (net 11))
 (segment (start 152.4 106.68) (end 152.4 101.6) (width 0.25) (layer F.Cu) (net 11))
 (segment (start 137.16 64.702081) (end 137.16 63.5) (width 0.25) (layer F.Cu) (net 11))
 (segment (start 137.16 97.79282) (end 137.16 64.702081) (width 0.25) (layer F.Cu) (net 11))
 (segment (start 140.96718 101.6) (end 137.16 97.79282) (width 0.25) (layer F.Cu) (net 11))
 (segment (start 152.4 101.6) (end 140.96718 101.6) (width 0.25) (layer F.Cu) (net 11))
 (segment (start 186.69 97.79) (end 186.69 101.6) (width 0.25) (layer F.Cu) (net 12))
 (segment (start 186.69 101.6) (end 157.48 101.6) (width 0.25) (layer F.Cu) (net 12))
 (segment (start 146.811999 97.028001) (end 146.05 97.79) (width 0.25) (layer F.Cu) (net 12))
 (segment (start 148.037019 95.802981) (end 146.811999 97.028001) (width 0.25) (layer F.Cu) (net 12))
 (segment (start 154.564561 95.802981) (end 148.037019 95.802981) (width 0.25) (layer F.Cu) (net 12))
 (segment (start 157.48 98.718418) (end 154.564561 95.802981) (width 0.25) (layer F.Cu) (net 12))
 (segment (start 157.48 101.6) (end 157.48 98.718418) (width 0.25) (layer F.Cu) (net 12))
 (segment (start 144.78 99.06) (end 139.7 99.06) (width 0.25) (layer F.Cu) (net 12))
 (segment (start 146.05 97.79) (end 144.78 99.06) (width 0.25) (layer F.Cu) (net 12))
 (segment (start 139.7 99.06) (end 138.43 97.79) (width 0.25) (layer F.Cu) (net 12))
 (segment (start 142.24 64.702081) (end 142.24 63.5) (width 0.25) (layer F.Cu) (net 12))
 (segment (start 142.24 86.018418) (end 142.24 64.702081) (width 0.25) (layer F.Cu) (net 12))
 (segment (start 138.43 89.828418) (end 142.24 86.018418) (width 0.25) (layer F.Cu) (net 12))
 (segment (start 138.43 97.79) (end 138.43 89.828418) (width 0.25) (layer F.Cu) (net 12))
 (segment (start 154.378162 96.25299) (end 156.21 98.084828) (width 0.25) (layer F.Cu) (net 13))
 (segment (start 148.59 97.79) (end 150.127011 96.252989) (width 0.25) (layer F.Cu) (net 13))
 (segment (start 150.127011 96.252989) (end 154.378162 96.25299) (width 0.25) (layer F.Cu) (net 13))
 (segment (start 156.21 98.084828) (end 156.21 102.87) (width 0.25) (layer F.Cu) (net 13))
 (segment (start 156.21 102.87) (end 189.23 102.87) (width 0.25) (layer F.Cu) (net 13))
 (segment (start 189.23 102.87) (end 189.23 97.79) (width 0.25) (layer F.Cu) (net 13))
 (segment (start 144.78 60.96) (end 144.78 54.61) (width 0.25) (layer F.Cu) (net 13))
 (segment (start 144.78 54.61) (end 191.77 54.61) (width 0.25) (layer F.Cu) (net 13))
 (segment (start 191.77 54.61) (end 191.77 83.82) (width 0.25) (layer F.Cu) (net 13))
 (segment (start 139.24999 89.644838) (end 139.24999 90.98999) (width 0.25) (layer F.Cu) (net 13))
 (segment (start 191.77 83.82) (end 145.074828 83.82) (width 0.25) (layer F.Cu) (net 13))
 (segment (start 145.074828 83.82) (end 139.24999 89.644838) (width 0.25) (layer F.Cu) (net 13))
 (segment (start 139.24999 90.98999) (end 142.24 93.98) (width 0.25) (layer F.Cu) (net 13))
 (segment (start 142.24 93.98) (end 189.23 93.98) (width 0.25) (layer F.Cu) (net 13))
 (segment (start 189.23 93.98) (end 189.23 97.79) (width 0.25) (layer F.Cu) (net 13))
 (segment (start 191.77 97.79) (end 191.77 104.14) (width 0.25) (layer F.Cu) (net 14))
 (segment (start 191.77 104.14) (end 154.94 104.14) (width 0.25) (layer F.Cu) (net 14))
 (segment (start 151.891999 97.028001) (end 151.13 97.79) (width 0.25) (layer F.Cu) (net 14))
 (segment (start 152.217001 96.702999) (end 151.891999 97.028001) (width 0.25) (layer F.Cu) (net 14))
 (segment (start 154.191761 96.702999) (end 152.217001 96.702999) (width 0.25) (layer F.Cu) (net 14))
 (segment (start 154.94 97.451238) (end 154.191761 96.702999) (width 0.25) (layer F.Cu) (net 14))
 (segment (start 154.94 104.14) (end 154.94 97.451238) (width 0.25) (layer F.Cu) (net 14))
 (segment (start 191.77 97.79) (end 191.77 92.71) (width 0.25) (layer F.Cu) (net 14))
 (segment (start 141.901238 92.71) (end 139.7 90.508762) (width 0.25) (layer F.Cu) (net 14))
 (segment (start 191.77 92.71) (end 141.901238 92.71) (width 0.25) (layer F.Cu) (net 14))
 (segment (start 139.7 89.831238) (end 144.441238 85.09) (width 0.25) (layer F.Cu) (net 14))
 (segment (start 139.7 90.508762) (end 139.7 89.831238) (width 0.25) (layer F.Cu) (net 14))
 (segment (start 144.441238 85.09) (end 193.04 85.09) (width 0.25) (layer F.Cu) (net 14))
 (segment (start 193.04 85.09) (end 193.04 53.34) (width 0.25) (layer F.Cu) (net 14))
 (segment (start 193.04 53.34) (end 142.24 53.34) (width 0.25) (layer F.Cu) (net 14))
 (segment (start 142.24 53.34) (end 142.24 60.96) (width 0.25) (layer F.Cu) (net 14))
 (segment (start 153.67 105.41) (end 194.31 105.41) (width 0.25) (layer F.Cu) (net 15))
 (segment (start 194.31 105.41) (end 194.31 97.79) (width 0.25) (layer F.Cu) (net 15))
 (segment (start 137.97999 97.9764) (end 137.97999 89.35001) (width 0.25) (layer F.Cu) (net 15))
 (segment (start 140.33359 100.33) (end 137.97999 97.9764) (width 0.25) (layer F.Cu) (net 15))
 (segment (start 153.67 100.33) (end 153.67 105.41) (width 0.25) (layer F.Cu) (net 15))
 (segment (start 153.67 100.33) (end 140.33359 100.33) (width 0.25) (layer F.Cu) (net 15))
 (segment (start 153.67 97.79) (end 153.67 100.33) (width 0.25) (layer F.Cu) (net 15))
 (segment (start 139.7 64.702081) (end 139.7 63.5) (width 0.25) (layer F.Cu) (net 15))
 (segment (start 139.7 87.63) (end 139.7 64.702081) (width 0.25) (layer F.Cu) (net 15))
 (segment (start 137.97999 89.35001) (end 139.7 87.63) (width 0.25) (layer F.Cu) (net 15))
 (segment (start 114.3 91.44) (end 114.3 97.79) (width 0.25) (layer F.Cu) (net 16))
 (segment (start 149.86 63.5) (end 149.86 74.93) (width 0.25) (layer B.Cu) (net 18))
 (segment (start 124.46 74.93) (end 122.681999 76.708001) (width 0.25) (layer B.Cu) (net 18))
 (segment (start 122.681999 76.708001) (end 121.92 77.47) (width 0.25) (layer B.Cu) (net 18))
 (segment (start 149.86 74.93) (end 124.46 74.93) (width 0.25) (layer B.Cu) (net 18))
 (segment (start 114.3 85.09) (end 114.3 77.47) (width 0.25) (layer F.Cu) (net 17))
 (segment (start 121.92 78.74) (end 121.92 91.44) (width 0.25) (layer B.Cu) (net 19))
 (segment (start 163.83 76.83641) (end 161.92641 78.74) (width 0.25) (layer B.Cu) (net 19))
 (segment (start 161.92641 78.74) (end 121.92 78.74) (width 0.25) (layer B.Cu) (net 19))
 (segment (start 162.56 60.96) (end 163.83 62.23) (width 0.25) (layer B.Cu) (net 19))
 (segment (start 163.83 62.23) (end 163.83 76.83641) (width 0.25) (layer B.Cu) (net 19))
 (segment (start 116.84 85.09) (end 116.84 97.79) (width 0.25) (layer F.Cu) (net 2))
 (segment (start 116.84 97.79) (end 116.84 104.14) (width 0.25) (layer F.Cu) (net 2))
 (segment (start 116.84 85.09) (end 116.84 67.31) (width 0.25) (layer F.Cu) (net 2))
 (segment (start 173.99 76.2) (end 170.18 72.39) (width 0.25) (layer F.Cu) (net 2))
 (segment (start 170.18 72.39) (end 170.18 63.5) (width 0.25) (layer F.Cu) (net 2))
 (segment (start 148.59 76.2) (end 152.4 76.2) (width 0.25) (layer F.Cu) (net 2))
 (segment (start 152.4 76.2) (end 152.4 63.5) (width 0.25) (layer F.Cu) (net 2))
 (segment (start 135.469999 64.349999) (end 134.62 63.5) (width 0.25) (layer F.Cu) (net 2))
 (segment (start 135.89 64.77) (end 135.469999 64.349999) (width 0.25) (layer F.Cu) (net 2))
 (segment (start 135.89 76.2) (end 135.89 64.77) (width 0.25) (layer F.Cu) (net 2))
 (segment (start 116.84 67.31) (end 135.89 67.31) (width 0.25) (layer F.Cu) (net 2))
 (segment (start 152.4 60.96) (end 152.4 58.42) (width 0.25) (layer B.Cu) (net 25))
 (segment (start 152.4 58.42) (end 119.38 58.42) (width 0.25) (layer B.Cu) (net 25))
 (segment (start 119.38 58.42) (end 119.38 64.77) (width 0.25) (layer B.Cu) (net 25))
 (segment (start 119.38 64.77) (end 116.84 64.77) (width 0.25) (layer B.Cu) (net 25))
 (segment (start 116.84 62.23) (end 116.84 57.15) (width 0.25) (layer B.Cu) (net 28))
 (segment (start 116.84 57.15) (end 157.48 57.15) (width 0.25) (layer B.Cu) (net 28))
 (segment (start 157.48 57.15) (end 157.48 60.96) (width 0.25) (layer B.Cu) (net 28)))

